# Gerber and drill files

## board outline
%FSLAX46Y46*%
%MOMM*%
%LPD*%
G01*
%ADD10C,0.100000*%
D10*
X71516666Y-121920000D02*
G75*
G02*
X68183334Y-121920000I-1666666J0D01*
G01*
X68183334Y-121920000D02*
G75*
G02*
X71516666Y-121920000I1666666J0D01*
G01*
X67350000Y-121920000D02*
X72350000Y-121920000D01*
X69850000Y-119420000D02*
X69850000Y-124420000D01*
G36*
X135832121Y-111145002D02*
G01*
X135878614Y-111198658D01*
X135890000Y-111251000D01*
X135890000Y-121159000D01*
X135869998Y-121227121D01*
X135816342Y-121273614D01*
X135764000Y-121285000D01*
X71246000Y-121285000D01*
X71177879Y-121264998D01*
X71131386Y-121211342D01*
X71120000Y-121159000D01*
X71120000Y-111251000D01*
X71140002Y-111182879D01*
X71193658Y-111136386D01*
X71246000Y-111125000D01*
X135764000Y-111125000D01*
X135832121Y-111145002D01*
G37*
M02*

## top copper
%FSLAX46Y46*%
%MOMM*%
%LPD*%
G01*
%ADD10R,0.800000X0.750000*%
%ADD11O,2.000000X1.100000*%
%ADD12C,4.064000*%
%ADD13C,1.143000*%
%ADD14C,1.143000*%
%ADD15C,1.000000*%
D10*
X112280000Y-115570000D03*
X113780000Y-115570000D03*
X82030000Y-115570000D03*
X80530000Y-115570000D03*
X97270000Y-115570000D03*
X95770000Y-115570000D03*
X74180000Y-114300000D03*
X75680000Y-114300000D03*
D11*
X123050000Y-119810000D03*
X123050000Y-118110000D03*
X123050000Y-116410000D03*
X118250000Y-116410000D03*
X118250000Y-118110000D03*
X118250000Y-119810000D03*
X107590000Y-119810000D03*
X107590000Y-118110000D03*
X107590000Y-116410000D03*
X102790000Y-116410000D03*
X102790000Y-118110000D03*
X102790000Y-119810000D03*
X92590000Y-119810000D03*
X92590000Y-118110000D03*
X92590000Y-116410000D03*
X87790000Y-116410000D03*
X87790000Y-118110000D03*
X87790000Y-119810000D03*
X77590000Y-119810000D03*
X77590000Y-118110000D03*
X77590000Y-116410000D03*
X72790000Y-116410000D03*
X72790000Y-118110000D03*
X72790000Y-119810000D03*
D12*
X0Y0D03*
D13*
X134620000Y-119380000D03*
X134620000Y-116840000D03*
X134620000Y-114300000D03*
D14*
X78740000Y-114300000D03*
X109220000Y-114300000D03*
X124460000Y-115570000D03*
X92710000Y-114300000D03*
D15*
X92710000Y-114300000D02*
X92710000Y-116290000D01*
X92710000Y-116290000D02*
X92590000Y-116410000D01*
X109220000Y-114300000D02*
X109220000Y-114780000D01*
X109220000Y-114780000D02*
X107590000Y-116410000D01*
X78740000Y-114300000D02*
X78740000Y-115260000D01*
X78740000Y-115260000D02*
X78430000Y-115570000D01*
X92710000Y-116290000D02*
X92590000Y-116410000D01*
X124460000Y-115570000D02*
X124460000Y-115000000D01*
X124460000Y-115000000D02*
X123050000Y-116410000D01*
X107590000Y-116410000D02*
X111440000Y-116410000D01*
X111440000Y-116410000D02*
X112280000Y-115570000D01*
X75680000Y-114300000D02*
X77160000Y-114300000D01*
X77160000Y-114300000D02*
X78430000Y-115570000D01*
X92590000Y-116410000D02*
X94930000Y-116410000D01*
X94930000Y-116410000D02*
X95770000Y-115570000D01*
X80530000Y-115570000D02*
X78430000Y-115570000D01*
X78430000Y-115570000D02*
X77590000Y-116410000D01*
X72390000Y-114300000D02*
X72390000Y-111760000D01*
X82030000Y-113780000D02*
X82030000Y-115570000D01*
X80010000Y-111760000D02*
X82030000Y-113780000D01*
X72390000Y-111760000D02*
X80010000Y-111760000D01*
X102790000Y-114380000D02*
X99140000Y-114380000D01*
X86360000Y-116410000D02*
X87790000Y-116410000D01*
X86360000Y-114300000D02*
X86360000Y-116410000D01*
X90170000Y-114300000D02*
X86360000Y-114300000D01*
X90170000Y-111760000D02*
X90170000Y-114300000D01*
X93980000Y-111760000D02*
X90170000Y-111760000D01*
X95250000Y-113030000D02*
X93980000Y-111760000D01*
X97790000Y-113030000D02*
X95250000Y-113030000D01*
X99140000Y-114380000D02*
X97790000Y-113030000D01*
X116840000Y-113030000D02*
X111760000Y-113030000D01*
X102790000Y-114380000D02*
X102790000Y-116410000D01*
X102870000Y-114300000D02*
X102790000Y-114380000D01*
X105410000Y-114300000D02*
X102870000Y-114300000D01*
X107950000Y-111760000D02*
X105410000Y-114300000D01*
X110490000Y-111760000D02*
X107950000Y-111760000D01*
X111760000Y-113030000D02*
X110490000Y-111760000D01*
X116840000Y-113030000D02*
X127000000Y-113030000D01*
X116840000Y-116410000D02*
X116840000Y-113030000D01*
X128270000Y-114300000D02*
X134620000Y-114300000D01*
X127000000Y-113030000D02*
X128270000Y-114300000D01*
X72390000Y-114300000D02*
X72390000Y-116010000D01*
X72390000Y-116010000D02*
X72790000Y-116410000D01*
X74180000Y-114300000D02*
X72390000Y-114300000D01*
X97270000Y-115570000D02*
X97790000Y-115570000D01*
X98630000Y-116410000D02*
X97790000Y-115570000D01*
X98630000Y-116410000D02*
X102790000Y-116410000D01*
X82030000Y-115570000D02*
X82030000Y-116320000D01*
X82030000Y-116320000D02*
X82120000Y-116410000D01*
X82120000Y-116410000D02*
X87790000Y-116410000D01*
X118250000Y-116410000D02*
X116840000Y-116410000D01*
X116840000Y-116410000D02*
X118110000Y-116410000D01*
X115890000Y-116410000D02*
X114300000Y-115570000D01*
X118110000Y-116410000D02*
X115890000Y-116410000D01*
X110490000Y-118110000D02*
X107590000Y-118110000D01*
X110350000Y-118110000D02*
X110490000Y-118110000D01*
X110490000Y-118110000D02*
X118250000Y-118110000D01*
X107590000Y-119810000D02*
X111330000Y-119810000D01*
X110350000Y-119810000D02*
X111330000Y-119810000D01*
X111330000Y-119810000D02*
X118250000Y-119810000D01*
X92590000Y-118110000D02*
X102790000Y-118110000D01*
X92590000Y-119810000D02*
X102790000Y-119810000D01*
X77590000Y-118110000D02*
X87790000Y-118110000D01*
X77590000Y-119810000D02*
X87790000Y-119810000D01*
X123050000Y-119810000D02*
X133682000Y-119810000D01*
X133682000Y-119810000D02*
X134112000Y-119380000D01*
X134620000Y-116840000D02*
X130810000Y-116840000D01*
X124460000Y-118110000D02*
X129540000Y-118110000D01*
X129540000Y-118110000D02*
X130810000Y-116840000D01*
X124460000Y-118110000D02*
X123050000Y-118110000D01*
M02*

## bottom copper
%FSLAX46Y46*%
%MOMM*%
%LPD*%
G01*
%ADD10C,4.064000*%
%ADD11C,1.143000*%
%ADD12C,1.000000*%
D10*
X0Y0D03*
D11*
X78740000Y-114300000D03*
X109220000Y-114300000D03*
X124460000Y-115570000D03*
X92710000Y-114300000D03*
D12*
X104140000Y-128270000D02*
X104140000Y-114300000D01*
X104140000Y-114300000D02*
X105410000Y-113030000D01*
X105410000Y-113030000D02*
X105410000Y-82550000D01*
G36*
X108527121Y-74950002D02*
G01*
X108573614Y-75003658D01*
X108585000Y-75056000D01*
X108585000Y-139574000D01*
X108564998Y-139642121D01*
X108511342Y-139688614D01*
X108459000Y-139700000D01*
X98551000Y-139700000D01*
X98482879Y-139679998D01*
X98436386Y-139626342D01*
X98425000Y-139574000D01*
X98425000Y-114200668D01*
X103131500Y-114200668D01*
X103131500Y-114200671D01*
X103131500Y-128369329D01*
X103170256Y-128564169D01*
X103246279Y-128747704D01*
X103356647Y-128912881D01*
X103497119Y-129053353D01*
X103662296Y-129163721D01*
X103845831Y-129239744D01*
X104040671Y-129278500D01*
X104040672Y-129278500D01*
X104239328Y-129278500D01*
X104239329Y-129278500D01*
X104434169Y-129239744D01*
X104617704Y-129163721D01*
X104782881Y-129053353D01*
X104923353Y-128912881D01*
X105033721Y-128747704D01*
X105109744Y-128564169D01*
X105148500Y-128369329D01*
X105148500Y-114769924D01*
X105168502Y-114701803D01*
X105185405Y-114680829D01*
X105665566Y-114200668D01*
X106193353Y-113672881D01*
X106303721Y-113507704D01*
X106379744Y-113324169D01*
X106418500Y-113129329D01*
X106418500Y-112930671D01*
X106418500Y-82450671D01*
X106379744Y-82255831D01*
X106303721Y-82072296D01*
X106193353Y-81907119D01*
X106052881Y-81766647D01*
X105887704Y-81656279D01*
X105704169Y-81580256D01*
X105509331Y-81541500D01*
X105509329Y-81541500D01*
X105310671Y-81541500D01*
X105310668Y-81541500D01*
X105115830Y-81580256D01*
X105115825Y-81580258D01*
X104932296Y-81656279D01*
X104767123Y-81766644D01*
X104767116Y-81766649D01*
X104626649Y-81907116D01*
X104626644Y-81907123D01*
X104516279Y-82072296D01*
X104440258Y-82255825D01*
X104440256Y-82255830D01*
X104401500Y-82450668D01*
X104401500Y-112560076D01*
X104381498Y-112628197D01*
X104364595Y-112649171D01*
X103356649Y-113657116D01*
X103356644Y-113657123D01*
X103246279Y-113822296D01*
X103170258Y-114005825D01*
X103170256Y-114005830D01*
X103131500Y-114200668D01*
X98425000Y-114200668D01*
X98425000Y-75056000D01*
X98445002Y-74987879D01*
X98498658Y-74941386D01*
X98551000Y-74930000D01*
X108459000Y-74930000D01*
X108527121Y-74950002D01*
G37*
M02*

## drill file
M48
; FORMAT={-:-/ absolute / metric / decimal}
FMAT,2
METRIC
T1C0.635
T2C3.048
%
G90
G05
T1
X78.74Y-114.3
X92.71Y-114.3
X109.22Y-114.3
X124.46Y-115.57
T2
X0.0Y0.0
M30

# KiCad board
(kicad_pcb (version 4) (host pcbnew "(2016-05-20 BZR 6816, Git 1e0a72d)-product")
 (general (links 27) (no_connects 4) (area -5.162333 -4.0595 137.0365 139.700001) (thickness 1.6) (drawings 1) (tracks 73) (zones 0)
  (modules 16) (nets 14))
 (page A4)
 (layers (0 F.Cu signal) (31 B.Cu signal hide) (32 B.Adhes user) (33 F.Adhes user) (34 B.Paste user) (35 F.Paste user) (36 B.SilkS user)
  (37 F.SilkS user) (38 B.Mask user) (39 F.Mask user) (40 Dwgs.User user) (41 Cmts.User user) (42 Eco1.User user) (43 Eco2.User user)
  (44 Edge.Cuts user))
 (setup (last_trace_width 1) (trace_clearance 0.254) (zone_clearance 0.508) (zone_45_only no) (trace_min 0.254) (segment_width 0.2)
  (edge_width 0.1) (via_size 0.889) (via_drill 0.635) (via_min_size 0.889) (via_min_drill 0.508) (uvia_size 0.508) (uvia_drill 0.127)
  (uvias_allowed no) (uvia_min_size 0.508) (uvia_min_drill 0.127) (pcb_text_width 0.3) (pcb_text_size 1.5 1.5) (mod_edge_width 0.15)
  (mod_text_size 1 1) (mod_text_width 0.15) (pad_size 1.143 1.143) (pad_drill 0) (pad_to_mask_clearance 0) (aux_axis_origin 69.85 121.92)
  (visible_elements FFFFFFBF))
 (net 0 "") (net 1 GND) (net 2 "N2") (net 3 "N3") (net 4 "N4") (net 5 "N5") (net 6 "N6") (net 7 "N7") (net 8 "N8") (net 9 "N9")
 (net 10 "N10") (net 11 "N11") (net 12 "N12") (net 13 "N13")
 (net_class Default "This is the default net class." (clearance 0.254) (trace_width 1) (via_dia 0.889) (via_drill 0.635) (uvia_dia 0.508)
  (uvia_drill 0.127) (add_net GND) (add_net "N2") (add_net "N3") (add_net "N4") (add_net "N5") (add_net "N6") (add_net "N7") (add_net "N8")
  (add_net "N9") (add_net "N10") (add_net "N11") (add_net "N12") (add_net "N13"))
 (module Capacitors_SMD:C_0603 (layer F.Cu) (at 113.03 115.57)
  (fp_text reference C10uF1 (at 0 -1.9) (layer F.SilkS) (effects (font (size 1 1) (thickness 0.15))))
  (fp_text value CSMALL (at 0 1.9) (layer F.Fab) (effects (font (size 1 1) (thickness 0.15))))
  (pad 1 smd rect (at -0.75 0) (size 0.8 0.75) (layers F.Cu F.Paste F.Mask) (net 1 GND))
  (pad 2 smd rect (at 0.75 0) (size 0.8 0.75) (layers F.Cu F.Paste F.Mask) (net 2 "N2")))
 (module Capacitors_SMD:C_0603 (layer F.Cu) (at 81.28 115.57 180)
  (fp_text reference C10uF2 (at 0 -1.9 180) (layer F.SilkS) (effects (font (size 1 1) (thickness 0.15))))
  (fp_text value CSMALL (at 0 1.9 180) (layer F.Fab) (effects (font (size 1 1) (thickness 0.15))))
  (pad 1 smd rect (at -0.75 0 180) (size 0.8 0.75) (layers F.Cu F.Paste F.Mask) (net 2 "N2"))
  (pad 2 smd rect (at 0.75 0 180) (size 0.8 0.75) (layers F.Cu F.Paste F.Mask) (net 1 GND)))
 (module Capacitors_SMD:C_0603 (layer F.Cu) (at 96.52 115.57 180)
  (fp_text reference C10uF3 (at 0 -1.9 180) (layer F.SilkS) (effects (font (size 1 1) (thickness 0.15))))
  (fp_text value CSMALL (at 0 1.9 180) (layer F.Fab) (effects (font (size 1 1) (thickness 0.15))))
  (pad 1 smd rect (at -0.75 0 180) (size 0.8 0.75) (layers F.Cu F.Paste F.Mask) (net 2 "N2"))
  (pad 2 smd rect (at 0.75 0 180) (size 0.8 0.75) (layers F.Cu F.Paste F.Mask) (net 1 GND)))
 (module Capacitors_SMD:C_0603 (layer F.Cu) (at 74.93 114.3)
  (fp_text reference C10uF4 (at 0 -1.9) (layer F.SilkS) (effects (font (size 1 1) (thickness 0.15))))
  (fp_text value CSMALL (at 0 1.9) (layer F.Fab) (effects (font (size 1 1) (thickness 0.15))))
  (pad 1 smd rect (at -0.75 0) (size 0.8 0.75) (layers F.Cu F.Paste F.Mask) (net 2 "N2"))
  (pad 2 smd rect (at 0.75 0) (size 0.8 0.75) (layers F.Cu F.Paste F.Mask) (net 1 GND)))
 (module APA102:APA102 (layer F.Cu) (at 120.65 118.11)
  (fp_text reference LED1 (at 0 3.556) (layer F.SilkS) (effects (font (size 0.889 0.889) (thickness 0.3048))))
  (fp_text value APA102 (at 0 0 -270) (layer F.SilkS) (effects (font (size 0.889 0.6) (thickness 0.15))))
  (pad 1 smd oval (at 2.4 1.7) (size 2 1.1) (layers F.Cu F.Paste F.Mask) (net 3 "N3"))
  (pad 2 smd oval (at 2.4 0) (size 2 1.1) (layers F.Cu F.Paste F.Mask) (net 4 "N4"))
  (pad 3 smd oval (at 2.4 -1.7) (size 2 1.1) (layers F.Cu F.Paste F.Mask) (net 1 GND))
  (pad 4 smd oval (at -2.4 -1.7 180) (size 2 1.1) (layers F.Cu F.Paste F.Mask) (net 2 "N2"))
  (pad 5 smd oval (at -2.4 0 180) (size 2 1.1) (layers F.Cu F.Paste F.Mask) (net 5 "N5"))
  (pad 6 smd oval (at -2.4 1.7 180) (size 2 1.1) (layers F.Cu F.Paste F.Mask) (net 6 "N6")))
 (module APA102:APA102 (layer F.Cu) (at 105.19 118.11)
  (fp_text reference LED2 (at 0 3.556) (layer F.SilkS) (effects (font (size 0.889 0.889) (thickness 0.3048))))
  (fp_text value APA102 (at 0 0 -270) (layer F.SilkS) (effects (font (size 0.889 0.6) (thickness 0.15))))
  (pad 1 smd oval (at 2.4 1.7) (size 2 1.1) (layers F.Cu F.Paste F.Mask) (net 6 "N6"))
  (pad 2 smd oval (at 2.4 0) (size 2 1.1) (layers F.Cu F.Paste F.Mask) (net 5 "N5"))
  (pad 3 smd oval (at 2.4 -1.7) (size 2 1.1) (layers F.Cu F.Paste F.Mask) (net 1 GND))
  (pad 4 smd oval (at -2.4 -1.7 180) (size 2 1.1) (layers F.Cu F.Paste F.Mask) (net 2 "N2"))
  (pad 5 smd oval (at -2.4 0 180) (size 2 1.1) (layers F.Cu F.Paste F.Mask) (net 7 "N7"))
  (pad 6 smd oval (at -2.4 1.7 180) (size 2 1.1) (layers F.Cu F.Paste F.Mask) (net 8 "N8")))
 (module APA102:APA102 (layer F.Cu) (at 90.19 118.11)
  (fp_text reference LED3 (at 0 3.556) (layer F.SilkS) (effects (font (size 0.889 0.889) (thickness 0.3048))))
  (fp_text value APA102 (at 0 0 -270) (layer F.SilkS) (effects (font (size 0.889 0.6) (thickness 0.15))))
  (pad 1 smd oval (at 2.4 1.7) (size 2 1.1) (layers F.Cu F.Paste F.Mask) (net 8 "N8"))
  (pad 2 smd oval (at 2.4 0) (size 2 1.1) (layers F.Cu F.Paste F.Mask) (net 7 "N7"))
  (pad 3 smd oval (at 2.4 -1.7) (size 2 1.1) (layers F.Cu F.Paste F.Mask) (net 1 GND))
  (pad 4 smd oval (at -2.4 -1.7 180) (size 2 1.1) (layers F.Cu F.Paste F.Mask) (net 2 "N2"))
  (pad 5 smd oval (at -2.4 0 180) (size 2 1.1) (layers F.Cu F.Paste F.Mask) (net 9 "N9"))
  (pad 6 smd oval (at -2.4 1.7 180) (size 2 1.1) (layers F.Cu F.Paste F.Mask) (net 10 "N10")))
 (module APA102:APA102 (layer F.Cu) (at 75.19 118.11)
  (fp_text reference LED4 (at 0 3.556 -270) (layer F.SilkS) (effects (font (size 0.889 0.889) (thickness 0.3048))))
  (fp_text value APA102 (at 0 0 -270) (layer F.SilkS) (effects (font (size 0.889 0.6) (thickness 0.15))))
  (pad 1 smd oval (at 2.4 1.7) (size 2 1.1) (layers F.Cu F.Paste F.Mask) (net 10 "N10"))
  (pad 2 smd oval (at 2.4 0) (size 2 1.1) (layers F.Cu F.Paste F.Mask) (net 9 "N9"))
  (pad 3 smd oval (at 2.4 -1.7) (size 2 1.1) (layers F.Cu F.Paste F.Mask) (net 1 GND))
  (pad 4 smd oval (at -2.4 -1.7 180) (size 2 1.1) (layers F.Cu F.Paste F.Mask) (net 2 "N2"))
  (pad 5 smd oval (at -2.4 0 180) (size 2 1.1) (layers F.Cu F.Paste F.Mask) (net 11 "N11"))
  (pad 6 smd oval (at -2.4 1.7 180) (size 2 1.1) (layers F.Cu F.Paste F.Mask) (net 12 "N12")))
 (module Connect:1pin (layer F.Cu) (at 0 0)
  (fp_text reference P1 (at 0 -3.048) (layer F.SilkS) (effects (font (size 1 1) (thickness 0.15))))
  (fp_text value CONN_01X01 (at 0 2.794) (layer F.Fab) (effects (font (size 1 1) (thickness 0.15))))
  (pad 1 thru_hole circle (at 0 0) (size 4.064 4.064) (drill 3.048) (layers *.Cu *.Mask F.SilkS) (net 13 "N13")))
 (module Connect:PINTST (layer F.Cu) (at 134.62 119.38 90)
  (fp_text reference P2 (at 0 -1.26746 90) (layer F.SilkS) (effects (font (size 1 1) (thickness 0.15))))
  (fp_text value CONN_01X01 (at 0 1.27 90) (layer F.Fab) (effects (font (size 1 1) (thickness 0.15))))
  (pad 1 smd circle (at 0 0 90) (size 1.143 1.143) (layers F.Cu F.Paste F.Mask) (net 3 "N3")))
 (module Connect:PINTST (layer F.Cu) (at 134.62 116.84 90)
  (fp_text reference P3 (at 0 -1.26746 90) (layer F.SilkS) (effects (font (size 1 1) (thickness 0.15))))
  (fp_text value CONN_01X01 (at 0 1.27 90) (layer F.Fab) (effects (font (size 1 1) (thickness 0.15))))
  (pad 1 smd circle (at 0 0 90) (size 1.143 1.143) (layers F.Cu F.Paste F.Mask) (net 4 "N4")))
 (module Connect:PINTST (layer F.Cu) (at 134.62 114.3 90)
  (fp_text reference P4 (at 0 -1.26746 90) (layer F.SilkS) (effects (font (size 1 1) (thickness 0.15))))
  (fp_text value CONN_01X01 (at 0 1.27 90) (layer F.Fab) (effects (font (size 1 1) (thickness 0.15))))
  (pad 1 smd circle (at 0 0 90) (size 1.143 1.143) (layers F.Cu F.Paste F.Mask) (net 2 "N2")))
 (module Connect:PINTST (layer F.Cu) (at 78.74 114.3 90)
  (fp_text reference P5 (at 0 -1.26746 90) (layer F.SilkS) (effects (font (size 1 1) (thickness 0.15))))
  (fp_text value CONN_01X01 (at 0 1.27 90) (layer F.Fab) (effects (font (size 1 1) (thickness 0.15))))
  (pad 1 thru_hole circle (at 0 0 90) (size 1.143 1.143) (drill 0.635) (layers *.Cu *.Mask F.SilkS) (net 1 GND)))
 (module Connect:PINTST (layer F.Cu) (at 109.22 114.3 90)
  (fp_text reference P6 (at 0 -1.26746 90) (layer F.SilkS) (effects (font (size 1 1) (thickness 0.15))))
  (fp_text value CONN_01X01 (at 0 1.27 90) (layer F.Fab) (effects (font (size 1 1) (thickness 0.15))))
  (pad 1 thru_hole circle (at 0 0 90) (size 1.143 1.143) (drill 0.635) (layers *.Cu *.Mask F.SilkS) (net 1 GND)))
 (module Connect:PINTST (layer F.Cu) (at 124.46 115.57 90)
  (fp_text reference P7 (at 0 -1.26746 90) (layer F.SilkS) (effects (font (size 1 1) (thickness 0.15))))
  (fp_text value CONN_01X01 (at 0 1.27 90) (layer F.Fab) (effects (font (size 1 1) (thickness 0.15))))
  (pad 1 thru_hole circle (at 0 0 90) (size 1.143 1.143) (drill 0.635) (layers *.Cu *.Mask F.SilkS) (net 1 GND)))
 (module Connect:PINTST (layer F.Cu) (at 92.71 114.3 90)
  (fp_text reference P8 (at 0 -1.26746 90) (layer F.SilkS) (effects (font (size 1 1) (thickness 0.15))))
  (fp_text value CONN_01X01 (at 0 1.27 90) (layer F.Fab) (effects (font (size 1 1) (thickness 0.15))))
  (pad 1 thru_hole circle (at 0 0 90) (size 1.143 1.143) (drill 0.635) (layers *.Cu *.Mask F.SilkS) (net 1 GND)))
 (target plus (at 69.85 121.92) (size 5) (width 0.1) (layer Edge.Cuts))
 (segment (start 104.14 128.27) (end 104.14 114.3) (width 1) (layer B.Cu) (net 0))
 (segment (start 104.14 114.3) (end 105.41 113.03) (width 1) (layer B.Cu) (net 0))
 (segment (start 105.41 113.03) (end 105.41 82.55) (width 1) (layer B.Cu) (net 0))
 (segment (start 92.71 114.3) (end 92.71 116.29) (width 1) (layer F.Cu) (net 1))
 (segment (start 92.71 116.29) (end 92.59 116.41) (width 1) (layer F.Cu) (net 1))
 (segment (start 109.22 114.3) (end 109.22 114.78) (width 1) (layer F.Cu) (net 1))
 (segment (start 109.22 114.78) (end 107.59 116.41) (width 1) (layer F.Cu) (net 1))
 (segment (start 78.74 114.3) (end 78.74 115.26) (width 1) (layer F.Cu) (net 1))
 (segment (start 78.74 115.26) (end 78.43 115.57) (width 1) (layer F.Cu) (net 1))
 (segment (start 92.71 116.29) (end 92.59 116.41) (width 1) (layer F.Cu) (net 1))
 (segment (start 124.46 115.57) (end 124.46 115) (width 1) (layer F.Cu) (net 1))
 (segment (start 124.46 115) (end 123.05 116.41) (width 1) (layer F.Cu) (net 1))
 (segment (start 107.59 116.41) (end 111.44 116.41) (width 1) (layer F.Cu) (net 1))
 (segment (start 111.44 116.41) (end 112.28 115.57) (width 1) (layer F.Cu) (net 1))
 (segment (start 75.68 114.3) (end 77.16 114.3) (width 1) (layer F.Cu) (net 1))
 (segment (start 77.16 114.3) (end 78.43 115.57) (width 1) (layer F.Cu) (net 1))
 (segment (start 92.59 116.41) (end 94.93 116.41) (width 1) (layer F.Cu) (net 1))
 (segment (start 94.93 116.41) (end 95.77 115.57) (width 1) (layer F.Cu) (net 1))
 (segment (start 80.53 115.57) (end 78.43 115.57) (width 1) (layer F.Cu) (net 1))
 (segment (start 78.43 115.57) (end 77.59 116.41) (width 1) (layer F.Cu) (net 1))
 (segment (start 72.39 114.3) (end 72.39 111.76) (width 1) (layer F.Cu) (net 2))
 (segment (start 82.03 113.78) (end 82.03 115.57) (width 1) (layer F.Cu) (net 2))
 (segment (start 80.01 111.76) (end 82.03 113.78) (width 1) (layer F.Cu) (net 2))
 (segment (start 72.39 111.76) (end 80.01 111.76) (width 1) (layer F.Cu) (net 2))
 (segment (start 102.79 114.38) (end 99.14 114.38) (width 1) (layer F.Cu) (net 2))
 (segment (start 86.36 116.41) (end 87.79 116.41) (width 1) (layer F.Cu) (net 2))
 (segment (start 86.36 114.3) (end 86.36 116.41) (width 1) (layer F.Cu) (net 2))
 (segment (start 90.17 114.3) (end 86.36 114.3) (width 1) (layer F.Cu) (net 2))
 (segment (start 90.17 111.76) (end 90.17 114.3) (width 1) (layer F.Cu) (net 2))
 (segment (start 93.98 111.76) (end 90.17 111.76) (width 1) (layer F.Cu) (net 2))
 (segment (start 95.25 113.03) (end 93.98 111.76) (width 1) (layer F.Cu) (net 2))
 (segment (start 97.79 113.03) (end 95.25 113.03) (width 1) (layer F.Cu) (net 2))
 (segment (start 99.14 114.38) (end 97.79 113.03) (width 1) (layer F.Cu) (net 2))
 (segment (start 116.84 113.03) (end 111.76 113.03) (width 1) (layer F.Cu) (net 2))
 (segment (start 102.79 114.38) (end 102.79 116.41) (width 1) (layer F.Cu) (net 2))
 (segment (start 102.87 114.3) (end 102.79 114.38) (width 1) (layer F.Cu) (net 2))
 (segment (start 105.41 114.3) (end 102.87 114.3) (width 1) (layer F.Cu) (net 2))
 (segment (start 107.95 111.76) (end 105.41 114.3) (width 1) (layer F.Cu) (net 2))
 (segment (start 110.49 111.76) (end 107.95 111.76) (width 1) (layer F.Cu) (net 2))
 (segment (start 111.76 113.03) (end 110.49 111.76) (width 1) (layer F.Cu) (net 2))
 (segment (start 116.84 113.03) (end 127 113.03) (width 1) (layer F.Cu) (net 2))
 (segment (start 116.84 116.41) (end 116.84 113.03) (width 1) (layer F.Cu) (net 2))
 (segment (start 128.27 114.3) (end 134.62 114.3) (width 1) (layer F.Cu) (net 2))
 (segment (start 127 113.03) (end 128.27 114.3) (width 1) (layer F.Cu) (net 2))
 (segment (start 72.39 114.3) (end 72.39 116.01) (width 1) (layer F.Cu) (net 2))
 (segment (start 72.39 116.01) (end 72.79 116.41) (width 1) (layer F.Cu) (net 2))
 (segment (start 74.18 114.3) (end 72.39 114.3) (width 1) (layer F.Cu) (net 2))
 (segment (start 97.27 115.57) (end 97.79 115.57) (width 1) (layer F.Cu) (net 2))
 (segment (start 98.63 116.41) (end 97.79 115.57) (width 1) (layer F.Cu) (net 2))
 (segment (start 98.63 116.41) (end 102.79 116.41) (width 1) (layer F.Cu) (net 2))
 (segment (start 82.03 115.57) (end 82.03 116.32) (width 1) (layer F.Cu) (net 2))
 (segment (start 82.03 116.32) (end 82.12 116.41) (width 1) (layer F.Cu) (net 2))
 (segment (start 82.12 116.41) (end 87.79 116.41) (width 1) (layer F.Cu) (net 2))
 (segment (start 118.25 116.41) (end 116.84 116.41) (width 1) (layer F.Cu) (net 2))
 (segment (start 116.84 116.41) (end 118.11 116.41) (width 1) (layer F.Cu) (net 2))
 (segment (start 115.89 116.41) (end 114.3 115.57) (width 1) (layer F.Cu) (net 2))
 (segment (start 118.11 116.41) (end 115.89 116.41) (width 1) (layer F.Cu) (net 2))
 (segment (start 110.49 118.11) (end 107.59 118.11) (width 1) (layer F.Cu) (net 5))
 (segment (start 110.35 118.11) (end 110.49 118.11) (width 1) (layer F.Cu) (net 5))
 (segment (start 110.49 118.11) (end 118.25 118.11) (width 1) (layer F.Cu) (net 5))
 (segment (start 107.59 119.81) (end 111.33 119.81) (width 1) (layer F.Cu) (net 6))
 (segment (start 110.35 119.81) (end 111.33 119.81) (width 1) (layer F.Cu) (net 6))
 (segment (start 111.33 119.81) (end 118.25 119.81) (width 1) (layer F.Cu) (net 6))
 (segment (start 92.59 118.11) (end 102.79 118.11) (width 1) (layer F.Cu) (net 7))
 (segment (start 92.59 119.81) (end 102.79 119.81) (width 1) (layer F.Cu) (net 8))
 (segment (start 77.59 118.11) (end 87.79 118.11) (width 1) (layer F.Cu) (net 9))
 (segment (start 77.59 119.81) (end 87.79 119.81) (width 1) (layer F.Cu) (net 10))
 (segment (start 123.05 119.81) (end 133.682 119.81) (width 1) (layer F.Cu) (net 3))
 (segment (start 133.682 119.81) (end 134.112 119.38) (width 1) (layer F.Cu) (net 3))
 (segment (start 134.62 116.84) (end 130.81 116.84) (width 1) (layer F.Cu) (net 4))
 (segment (start 124.46 118.11) (end 129.54 118.11) (width 1) (layer F.Cu) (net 4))
 (segment (start 129.54 118.11) (end 130.81 116.84) (width 1) (layer F.Cu) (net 4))
 (segment (start 124.46 118.11) (end 123.05 118.11) (width 1) (layer F.Cu) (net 4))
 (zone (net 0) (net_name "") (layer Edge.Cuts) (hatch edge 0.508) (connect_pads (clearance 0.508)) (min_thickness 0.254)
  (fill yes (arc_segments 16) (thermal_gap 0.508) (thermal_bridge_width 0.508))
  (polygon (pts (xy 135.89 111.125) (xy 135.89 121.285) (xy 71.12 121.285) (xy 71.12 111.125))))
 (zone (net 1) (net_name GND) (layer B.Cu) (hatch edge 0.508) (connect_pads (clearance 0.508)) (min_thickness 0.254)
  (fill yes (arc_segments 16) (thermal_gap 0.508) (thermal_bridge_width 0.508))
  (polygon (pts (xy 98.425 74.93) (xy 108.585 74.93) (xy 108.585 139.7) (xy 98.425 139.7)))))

